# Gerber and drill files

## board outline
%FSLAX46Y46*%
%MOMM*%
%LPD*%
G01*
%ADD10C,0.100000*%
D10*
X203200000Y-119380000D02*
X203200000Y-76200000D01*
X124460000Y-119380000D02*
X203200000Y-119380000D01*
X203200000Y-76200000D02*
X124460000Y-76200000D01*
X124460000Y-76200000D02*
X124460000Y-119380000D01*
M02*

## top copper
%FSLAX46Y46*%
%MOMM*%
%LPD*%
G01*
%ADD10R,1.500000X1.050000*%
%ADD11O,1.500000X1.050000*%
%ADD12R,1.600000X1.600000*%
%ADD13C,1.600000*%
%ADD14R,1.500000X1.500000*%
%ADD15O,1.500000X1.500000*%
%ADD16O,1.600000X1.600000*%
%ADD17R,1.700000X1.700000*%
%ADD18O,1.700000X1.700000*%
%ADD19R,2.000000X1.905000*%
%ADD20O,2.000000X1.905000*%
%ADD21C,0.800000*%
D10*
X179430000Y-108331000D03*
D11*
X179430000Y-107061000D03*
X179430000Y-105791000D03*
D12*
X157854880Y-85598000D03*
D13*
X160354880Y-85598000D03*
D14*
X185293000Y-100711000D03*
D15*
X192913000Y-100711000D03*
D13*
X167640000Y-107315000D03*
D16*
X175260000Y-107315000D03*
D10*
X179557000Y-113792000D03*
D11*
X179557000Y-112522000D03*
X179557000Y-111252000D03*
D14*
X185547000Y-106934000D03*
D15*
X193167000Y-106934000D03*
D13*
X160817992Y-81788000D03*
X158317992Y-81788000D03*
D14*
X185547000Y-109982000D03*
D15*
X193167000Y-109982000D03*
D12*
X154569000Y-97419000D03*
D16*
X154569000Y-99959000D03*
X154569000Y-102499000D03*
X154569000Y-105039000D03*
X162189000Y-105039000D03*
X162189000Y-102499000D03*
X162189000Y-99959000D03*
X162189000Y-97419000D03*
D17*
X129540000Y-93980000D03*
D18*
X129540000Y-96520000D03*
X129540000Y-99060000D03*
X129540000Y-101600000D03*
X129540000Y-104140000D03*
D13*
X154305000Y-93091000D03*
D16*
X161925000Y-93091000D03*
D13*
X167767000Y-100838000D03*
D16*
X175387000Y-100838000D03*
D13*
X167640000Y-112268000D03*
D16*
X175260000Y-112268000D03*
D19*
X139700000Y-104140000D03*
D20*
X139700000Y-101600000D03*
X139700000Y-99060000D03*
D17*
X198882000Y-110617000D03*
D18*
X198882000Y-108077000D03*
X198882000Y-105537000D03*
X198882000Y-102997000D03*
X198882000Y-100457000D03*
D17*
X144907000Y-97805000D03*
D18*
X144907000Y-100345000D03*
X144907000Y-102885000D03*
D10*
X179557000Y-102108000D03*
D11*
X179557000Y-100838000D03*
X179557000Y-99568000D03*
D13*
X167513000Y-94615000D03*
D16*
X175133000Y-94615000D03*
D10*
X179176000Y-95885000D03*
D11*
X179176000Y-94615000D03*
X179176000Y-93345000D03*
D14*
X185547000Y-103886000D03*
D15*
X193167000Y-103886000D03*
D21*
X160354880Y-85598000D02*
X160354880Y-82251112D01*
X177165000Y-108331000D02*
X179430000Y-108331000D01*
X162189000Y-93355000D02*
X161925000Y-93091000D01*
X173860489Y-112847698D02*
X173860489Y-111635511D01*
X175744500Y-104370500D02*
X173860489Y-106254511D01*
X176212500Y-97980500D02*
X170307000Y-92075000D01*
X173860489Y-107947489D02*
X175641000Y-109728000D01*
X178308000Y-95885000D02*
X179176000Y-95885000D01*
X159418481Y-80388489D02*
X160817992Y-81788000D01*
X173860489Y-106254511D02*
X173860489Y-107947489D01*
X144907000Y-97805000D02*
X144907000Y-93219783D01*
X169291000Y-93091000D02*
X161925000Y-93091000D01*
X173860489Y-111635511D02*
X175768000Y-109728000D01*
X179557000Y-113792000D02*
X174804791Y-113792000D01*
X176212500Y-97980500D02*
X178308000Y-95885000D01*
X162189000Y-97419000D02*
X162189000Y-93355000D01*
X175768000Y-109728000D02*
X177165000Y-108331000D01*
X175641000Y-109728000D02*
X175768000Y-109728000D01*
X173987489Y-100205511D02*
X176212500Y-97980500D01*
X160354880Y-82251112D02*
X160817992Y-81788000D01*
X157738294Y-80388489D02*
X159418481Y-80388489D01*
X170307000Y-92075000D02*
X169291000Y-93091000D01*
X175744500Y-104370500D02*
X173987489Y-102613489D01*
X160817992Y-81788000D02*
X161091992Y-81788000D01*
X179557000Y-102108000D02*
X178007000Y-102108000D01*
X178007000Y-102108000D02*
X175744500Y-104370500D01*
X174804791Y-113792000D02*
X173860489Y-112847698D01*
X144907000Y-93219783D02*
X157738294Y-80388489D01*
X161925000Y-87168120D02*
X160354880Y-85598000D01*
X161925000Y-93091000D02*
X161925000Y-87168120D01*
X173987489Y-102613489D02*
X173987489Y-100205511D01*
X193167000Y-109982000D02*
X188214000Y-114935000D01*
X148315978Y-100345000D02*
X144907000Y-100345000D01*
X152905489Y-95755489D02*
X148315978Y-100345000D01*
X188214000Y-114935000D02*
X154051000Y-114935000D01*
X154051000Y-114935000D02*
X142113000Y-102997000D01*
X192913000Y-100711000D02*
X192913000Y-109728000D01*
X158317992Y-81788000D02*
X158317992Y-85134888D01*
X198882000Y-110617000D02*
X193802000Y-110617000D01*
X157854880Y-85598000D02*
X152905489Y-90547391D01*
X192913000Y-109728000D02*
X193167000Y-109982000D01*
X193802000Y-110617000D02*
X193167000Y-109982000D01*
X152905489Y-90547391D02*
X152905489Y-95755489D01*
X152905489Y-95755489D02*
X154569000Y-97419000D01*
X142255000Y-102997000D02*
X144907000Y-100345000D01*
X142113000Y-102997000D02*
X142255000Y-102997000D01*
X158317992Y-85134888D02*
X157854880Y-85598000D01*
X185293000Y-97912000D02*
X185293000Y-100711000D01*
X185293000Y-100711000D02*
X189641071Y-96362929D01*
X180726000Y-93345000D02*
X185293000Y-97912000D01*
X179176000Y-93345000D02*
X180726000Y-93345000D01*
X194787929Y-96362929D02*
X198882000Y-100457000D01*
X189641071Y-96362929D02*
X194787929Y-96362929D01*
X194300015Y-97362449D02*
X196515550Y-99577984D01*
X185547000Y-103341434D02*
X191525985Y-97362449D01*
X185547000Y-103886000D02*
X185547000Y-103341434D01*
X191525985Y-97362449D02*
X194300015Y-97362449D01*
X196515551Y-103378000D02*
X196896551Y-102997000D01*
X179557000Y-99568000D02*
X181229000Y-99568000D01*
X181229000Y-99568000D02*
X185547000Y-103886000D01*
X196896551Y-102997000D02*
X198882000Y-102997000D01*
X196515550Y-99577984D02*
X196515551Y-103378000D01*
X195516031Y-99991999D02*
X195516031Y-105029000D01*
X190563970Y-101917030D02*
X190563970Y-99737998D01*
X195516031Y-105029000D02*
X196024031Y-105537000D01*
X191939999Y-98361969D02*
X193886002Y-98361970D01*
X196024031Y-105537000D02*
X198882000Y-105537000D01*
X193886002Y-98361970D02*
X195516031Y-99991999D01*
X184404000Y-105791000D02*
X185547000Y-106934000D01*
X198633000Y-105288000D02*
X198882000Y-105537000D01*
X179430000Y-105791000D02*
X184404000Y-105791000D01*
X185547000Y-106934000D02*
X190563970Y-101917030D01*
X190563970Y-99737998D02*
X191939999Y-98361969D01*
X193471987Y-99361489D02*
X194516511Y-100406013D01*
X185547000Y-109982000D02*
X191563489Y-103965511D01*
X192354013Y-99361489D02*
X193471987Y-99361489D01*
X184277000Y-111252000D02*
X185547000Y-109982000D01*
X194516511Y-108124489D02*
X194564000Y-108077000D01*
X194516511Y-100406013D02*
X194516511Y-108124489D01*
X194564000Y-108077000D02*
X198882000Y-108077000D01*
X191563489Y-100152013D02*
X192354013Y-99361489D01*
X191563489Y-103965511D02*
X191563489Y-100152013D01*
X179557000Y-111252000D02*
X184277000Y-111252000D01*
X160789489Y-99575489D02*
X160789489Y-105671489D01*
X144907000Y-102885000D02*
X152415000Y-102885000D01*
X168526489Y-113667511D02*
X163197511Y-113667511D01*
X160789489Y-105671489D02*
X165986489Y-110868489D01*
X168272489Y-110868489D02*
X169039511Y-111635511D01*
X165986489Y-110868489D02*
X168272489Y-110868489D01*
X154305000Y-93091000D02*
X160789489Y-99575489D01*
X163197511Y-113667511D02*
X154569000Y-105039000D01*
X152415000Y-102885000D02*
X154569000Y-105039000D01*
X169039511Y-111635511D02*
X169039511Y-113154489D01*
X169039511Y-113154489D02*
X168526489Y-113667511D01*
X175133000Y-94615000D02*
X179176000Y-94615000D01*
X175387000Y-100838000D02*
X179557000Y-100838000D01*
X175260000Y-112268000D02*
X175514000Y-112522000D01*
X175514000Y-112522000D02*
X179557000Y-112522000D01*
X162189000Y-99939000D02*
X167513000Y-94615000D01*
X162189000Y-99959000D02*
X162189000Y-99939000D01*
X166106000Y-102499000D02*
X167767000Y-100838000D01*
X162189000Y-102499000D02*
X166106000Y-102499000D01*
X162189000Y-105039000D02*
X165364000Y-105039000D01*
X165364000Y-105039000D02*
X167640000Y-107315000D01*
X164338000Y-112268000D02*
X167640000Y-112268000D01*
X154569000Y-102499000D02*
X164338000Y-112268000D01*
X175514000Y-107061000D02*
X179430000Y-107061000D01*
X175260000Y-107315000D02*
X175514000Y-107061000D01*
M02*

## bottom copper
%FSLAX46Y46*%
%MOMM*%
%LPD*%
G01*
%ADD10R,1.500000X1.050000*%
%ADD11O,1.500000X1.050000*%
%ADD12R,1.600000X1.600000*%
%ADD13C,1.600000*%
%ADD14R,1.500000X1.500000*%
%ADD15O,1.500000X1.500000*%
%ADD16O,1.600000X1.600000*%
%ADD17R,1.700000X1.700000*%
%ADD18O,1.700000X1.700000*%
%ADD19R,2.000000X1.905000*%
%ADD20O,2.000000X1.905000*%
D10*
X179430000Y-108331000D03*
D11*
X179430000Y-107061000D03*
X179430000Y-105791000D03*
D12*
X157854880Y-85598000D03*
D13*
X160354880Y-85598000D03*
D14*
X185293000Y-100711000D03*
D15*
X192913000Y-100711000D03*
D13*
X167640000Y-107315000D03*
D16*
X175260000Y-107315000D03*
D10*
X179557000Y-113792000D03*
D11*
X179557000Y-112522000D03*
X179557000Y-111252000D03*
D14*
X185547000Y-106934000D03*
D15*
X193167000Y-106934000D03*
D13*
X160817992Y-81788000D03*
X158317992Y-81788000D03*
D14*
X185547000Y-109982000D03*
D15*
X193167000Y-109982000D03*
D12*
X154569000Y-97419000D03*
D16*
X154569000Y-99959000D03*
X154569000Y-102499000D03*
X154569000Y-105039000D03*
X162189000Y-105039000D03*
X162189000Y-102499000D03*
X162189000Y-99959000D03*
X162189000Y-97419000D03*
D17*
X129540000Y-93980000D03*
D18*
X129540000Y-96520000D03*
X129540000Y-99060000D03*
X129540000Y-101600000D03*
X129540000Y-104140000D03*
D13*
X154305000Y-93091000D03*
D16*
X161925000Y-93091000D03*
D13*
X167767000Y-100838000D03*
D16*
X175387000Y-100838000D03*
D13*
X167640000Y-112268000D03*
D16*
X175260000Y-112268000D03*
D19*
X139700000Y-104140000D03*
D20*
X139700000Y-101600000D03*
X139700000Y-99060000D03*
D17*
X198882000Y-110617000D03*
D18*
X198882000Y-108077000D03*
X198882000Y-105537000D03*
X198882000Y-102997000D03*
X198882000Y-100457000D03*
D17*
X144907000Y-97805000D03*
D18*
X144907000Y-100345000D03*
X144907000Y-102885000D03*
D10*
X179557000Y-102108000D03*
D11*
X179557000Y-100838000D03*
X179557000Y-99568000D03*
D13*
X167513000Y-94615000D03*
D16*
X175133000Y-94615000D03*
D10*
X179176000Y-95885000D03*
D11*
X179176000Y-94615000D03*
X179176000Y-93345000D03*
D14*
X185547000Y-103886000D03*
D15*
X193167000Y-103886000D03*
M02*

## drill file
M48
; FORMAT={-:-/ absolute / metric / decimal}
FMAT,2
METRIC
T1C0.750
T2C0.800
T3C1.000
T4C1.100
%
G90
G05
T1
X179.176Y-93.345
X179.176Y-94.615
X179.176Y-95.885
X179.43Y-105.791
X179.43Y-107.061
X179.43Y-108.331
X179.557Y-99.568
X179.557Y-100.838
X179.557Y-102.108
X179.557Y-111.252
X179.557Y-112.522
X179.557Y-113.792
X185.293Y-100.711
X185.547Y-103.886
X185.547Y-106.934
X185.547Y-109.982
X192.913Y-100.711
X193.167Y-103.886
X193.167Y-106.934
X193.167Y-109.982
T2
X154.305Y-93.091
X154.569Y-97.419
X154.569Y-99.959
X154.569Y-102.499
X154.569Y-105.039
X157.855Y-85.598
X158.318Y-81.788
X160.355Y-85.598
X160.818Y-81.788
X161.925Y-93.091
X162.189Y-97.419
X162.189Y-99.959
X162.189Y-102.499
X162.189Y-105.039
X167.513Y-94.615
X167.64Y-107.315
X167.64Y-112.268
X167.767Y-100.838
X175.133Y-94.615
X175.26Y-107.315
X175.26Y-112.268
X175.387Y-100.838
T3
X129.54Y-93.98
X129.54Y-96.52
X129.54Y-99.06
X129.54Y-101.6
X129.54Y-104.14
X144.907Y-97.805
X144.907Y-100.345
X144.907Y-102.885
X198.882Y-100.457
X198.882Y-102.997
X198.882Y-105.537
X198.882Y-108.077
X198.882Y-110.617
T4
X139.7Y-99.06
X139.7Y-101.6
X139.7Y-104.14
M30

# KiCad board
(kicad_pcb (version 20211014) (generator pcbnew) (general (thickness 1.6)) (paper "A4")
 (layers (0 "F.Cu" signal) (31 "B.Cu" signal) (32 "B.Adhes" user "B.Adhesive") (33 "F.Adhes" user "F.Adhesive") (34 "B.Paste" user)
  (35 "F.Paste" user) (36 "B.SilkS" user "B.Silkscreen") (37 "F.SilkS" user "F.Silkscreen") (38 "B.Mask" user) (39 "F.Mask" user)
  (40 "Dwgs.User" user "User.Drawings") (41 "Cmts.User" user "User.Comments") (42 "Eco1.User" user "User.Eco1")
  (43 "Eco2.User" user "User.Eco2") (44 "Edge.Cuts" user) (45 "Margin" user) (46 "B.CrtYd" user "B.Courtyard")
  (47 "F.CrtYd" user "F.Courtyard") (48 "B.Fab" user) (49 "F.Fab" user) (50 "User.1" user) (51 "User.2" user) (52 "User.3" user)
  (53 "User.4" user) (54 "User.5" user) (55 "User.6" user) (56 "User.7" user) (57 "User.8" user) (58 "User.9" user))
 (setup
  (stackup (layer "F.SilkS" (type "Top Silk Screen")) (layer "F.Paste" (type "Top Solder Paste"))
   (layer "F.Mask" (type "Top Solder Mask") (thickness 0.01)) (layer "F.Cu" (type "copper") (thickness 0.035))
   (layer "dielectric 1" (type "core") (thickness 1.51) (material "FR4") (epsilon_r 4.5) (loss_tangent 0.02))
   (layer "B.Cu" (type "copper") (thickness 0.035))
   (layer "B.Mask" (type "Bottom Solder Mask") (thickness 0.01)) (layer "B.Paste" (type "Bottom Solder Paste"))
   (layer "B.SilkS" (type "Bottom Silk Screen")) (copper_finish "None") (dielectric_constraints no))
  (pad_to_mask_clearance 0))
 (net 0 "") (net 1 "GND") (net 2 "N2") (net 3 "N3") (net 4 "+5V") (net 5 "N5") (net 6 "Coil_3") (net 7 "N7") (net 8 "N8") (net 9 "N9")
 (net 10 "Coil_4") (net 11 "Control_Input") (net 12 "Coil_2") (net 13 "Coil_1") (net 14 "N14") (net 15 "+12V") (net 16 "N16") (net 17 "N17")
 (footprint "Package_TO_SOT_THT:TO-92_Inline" (layer "F.Cu") (at 179.43 108.331 90)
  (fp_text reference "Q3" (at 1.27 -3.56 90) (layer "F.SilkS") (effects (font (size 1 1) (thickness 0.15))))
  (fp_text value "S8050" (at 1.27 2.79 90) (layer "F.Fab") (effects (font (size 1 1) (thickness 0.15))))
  (pad "1" thru_hole rect (at 0 0 90) (size 1.05 1.5) (drill 0.75) (layers *.Cu *.Mask) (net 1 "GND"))
  (pad "2" thru_hole oval (at 1.27 0 90) (size 1.05 1.5) (drill 0.75) (layers *.Cu *.Mask) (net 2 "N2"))
  (pad "3" thru_hole oval (at 2.54 0 90) (size 1.05 1.5) (drill 0.75) (layers *.Cu *.Mask) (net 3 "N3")))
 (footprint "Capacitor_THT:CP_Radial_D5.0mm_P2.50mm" (layer "F.Cu") (at 157.85488 85.598)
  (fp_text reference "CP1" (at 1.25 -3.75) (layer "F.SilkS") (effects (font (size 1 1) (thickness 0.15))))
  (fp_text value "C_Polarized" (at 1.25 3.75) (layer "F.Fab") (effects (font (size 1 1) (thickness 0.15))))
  (pad "1" thru_hole rect (at 0 0) (size 1.6 1.6) (drill 0.8) (layers *.Cu *.Mask) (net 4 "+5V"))
  (pad "2" thru_hole circle (at 2.5 0) (size 1.6 1.6) (drill 0.8) (layers *.Cu *.Mask) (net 1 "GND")))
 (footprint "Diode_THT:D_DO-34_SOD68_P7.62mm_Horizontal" (layer "F.Cu") (at 185.293 100.711)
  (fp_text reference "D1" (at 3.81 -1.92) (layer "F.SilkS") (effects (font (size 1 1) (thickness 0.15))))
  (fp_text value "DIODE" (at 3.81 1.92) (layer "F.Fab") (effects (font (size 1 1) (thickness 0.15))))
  (pad "1" thru_hole rect (at 0 0) (size 1.5 1.5) (drill 0.75) (layers *.Cu *.Mask) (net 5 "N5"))
  (pad "2" thru_hole oval (at 7.62 0) (size 1.5 1.5) (drill 0.75) (layers *.Cu *.Mask) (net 4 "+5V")))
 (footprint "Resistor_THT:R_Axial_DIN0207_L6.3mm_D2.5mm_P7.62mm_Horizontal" (layer "F.Cu") (at 167.64 107.315)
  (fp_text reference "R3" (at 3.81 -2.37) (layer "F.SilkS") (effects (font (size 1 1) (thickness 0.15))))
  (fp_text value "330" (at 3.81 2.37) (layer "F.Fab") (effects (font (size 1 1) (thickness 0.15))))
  (pad "1" thru_hole circle (at 0 0) (size 1.6 1.6) (drill 0.8) (layers *.Cu *.Mask) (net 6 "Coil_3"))
  (pad "2" thru_hole oval (at 7.62 0) (size 1.6 1.6) (drill 0.8) (layers *.Cu *.Mask) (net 2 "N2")))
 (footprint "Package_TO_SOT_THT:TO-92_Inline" (layer "F.Cu") (at 179.557 113.792 90)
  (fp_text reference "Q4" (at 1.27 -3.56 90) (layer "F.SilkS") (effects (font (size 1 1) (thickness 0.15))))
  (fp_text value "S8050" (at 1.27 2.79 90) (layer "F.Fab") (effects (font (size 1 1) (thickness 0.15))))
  (pad "1" thru_hole rect (at 0 0 90) (size 1.05 1.5) (drill 0.75) (layers *.Cu *.Mask) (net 1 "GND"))
  (pad "2" thru_hole oval (at 1.27 0 90) (size 1.05 1.5) (drill 0.75) (layers *.Cu *.Mask) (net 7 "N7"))
  (pad "3" thru_hole oval (at 2.54 0 90) (size 1.05 1.5) (drill 0.75) (layers *.Cu *.Mask) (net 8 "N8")))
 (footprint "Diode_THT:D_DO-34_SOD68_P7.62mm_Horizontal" (layer "F.Cu") (at 185.547 106.934)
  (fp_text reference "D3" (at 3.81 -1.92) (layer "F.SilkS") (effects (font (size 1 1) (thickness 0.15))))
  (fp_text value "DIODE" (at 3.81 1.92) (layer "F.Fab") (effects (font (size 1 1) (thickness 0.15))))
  (pad "1" thru_hole rect (at 0 0) (size 1.5 1.5) (drill 0.75) (layers *.Cu *.Mask) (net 3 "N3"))
  (pad "2" thru_hole oval (at 7.62 0) (size 1.5 1.5) (drill 0.75) (layers *.Cu *.Mask) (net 4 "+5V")))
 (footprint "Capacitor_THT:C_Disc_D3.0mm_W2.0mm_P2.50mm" (layer "F.Cu") (at 160.817992 81.788 180)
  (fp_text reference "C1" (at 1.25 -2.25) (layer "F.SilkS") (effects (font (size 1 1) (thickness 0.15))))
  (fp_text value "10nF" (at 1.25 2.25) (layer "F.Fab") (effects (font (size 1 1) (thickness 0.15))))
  (pad "1" thru_hole circle (at 0 0 180) (size 1.6 1.6) (drill 0.8) (layers *.Cu *.Mask) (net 1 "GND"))
  (pad "2" thru_hole circle (at 2.5 0 180) (size 1.6 1.6) (drill 0.8) (layers *.Cu *.Mask) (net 4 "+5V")))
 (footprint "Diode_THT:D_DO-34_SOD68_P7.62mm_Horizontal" (layer "F.Cu") (at 185.547 109.982)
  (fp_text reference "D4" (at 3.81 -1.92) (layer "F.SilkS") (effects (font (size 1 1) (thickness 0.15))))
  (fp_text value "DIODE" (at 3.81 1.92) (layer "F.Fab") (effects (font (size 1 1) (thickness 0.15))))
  (pad "1" thru_hole rect (at 0 0) (size 1.5 1.5) (drill 0.75) (layers *.Cu *.Mask) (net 8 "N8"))
  (pad "2" thru_hole oval (at 7.62 0) (size 1.5 1.5) (drill 0.75) (layers *.Cu *.Mask) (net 4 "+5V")))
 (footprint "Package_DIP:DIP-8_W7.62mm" (layer "F.Cu") (at 154.569 97.419)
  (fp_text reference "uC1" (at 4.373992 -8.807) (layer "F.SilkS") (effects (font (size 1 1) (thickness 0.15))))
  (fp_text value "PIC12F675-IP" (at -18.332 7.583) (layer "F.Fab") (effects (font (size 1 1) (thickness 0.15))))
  (pad "1" thru_hole rect (at 0 0) (size 1.6 1.6) (drill 0.8) (layers *.Cu *.Mask) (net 4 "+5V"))
  (pad "2" thru_hole oval (at 0 2.54) (size 1.6 1.6) (drill 0.8) (layers *.Cu *.Mask) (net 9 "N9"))
  (pad "3" thru_hole oval (at 0 5.08) (size 1.6 1.6) (drill 0.8) (layers *.Cu *.Mask) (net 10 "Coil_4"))
  (pad "4" thru_hole oval (at 0 7.62) (size 1.6 1.6) (drill 0.8) (layers *.Cu *.Mask) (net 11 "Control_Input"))
  (pad "5" thru_hole oval (at 7.62 7.62) (size 1.6 1.6) (drill 0.8) (layers *.Cu *.Mask) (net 6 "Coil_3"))
  (pad "6" thru_hole oval (at 7.62 5.08) (size 1.6 1.6) (drill 0.8) (layers *.Cu *.Mask) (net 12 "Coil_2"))
  (pad "7" thru_hole oval (at 7.62 2.54) (size 1.6 1.6) (drill 0.8) (layers *.Cu *.Mask) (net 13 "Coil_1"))
  (pad "8" thru_hole oval (at 7.62 0) (size 1.6 1.6) (drill 0.8) (layers *.Cu *.Mask) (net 1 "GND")))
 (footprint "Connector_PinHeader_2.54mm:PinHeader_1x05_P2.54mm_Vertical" (layer "F.Cu") (at 129.54 93.98)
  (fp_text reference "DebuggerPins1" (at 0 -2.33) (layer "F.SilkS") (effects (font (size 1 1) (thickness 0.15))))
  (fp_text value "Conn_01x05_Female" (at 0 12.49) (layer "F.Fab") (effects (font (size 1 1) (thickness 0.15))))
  (pad "1" thru_hole rect (at 0 0) (size 1.7 1.7) (drill 1) (layers *.Cu *.Mask) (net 11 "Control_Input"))
  (pad "2" thru_hole oval (at 0 2.54) (size 1.7 1.7) (drill 1) (layers *.Cu *.Mask) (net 4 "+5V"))
  (pad "3" thru_hole oval (at 0 5.08) (size 1.7 1.7) (drill 1) (layers *.Cu *.Mask) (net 1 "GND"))
  (pad "4" thru_hole oval (at 0 7.62) (size 1.7 1.7) (drill 1) (layers *.Cu *.Mask) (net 13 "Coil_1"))
  (pad "5" thru_hole oval (at 0 10.16) (size 1.7 1.7) (drill 1) (layers *.Cu *.Mask) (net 12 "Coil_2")))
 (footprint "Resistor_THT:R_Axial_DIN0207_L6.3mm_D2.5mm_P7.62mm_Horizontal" (layer "F.Cu") (at 154.305 93.091)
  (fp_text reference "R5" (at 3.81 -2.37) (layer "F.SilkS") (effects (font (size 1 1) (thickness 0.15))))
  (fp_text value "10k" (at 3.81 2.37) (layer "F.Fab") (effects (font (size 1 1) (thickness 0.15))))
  (pad "1" thru_hole circle (at 0 0) (size 1.6 1.6) (drill 0.8) (layers *.Cu *.Mask) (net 1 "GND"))
  (pad "2" thru_hole oval (at 7.62 0) (size 1.6 1.6) (drill 0.8) (layers *.Cu *.Mask) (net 11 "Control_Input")))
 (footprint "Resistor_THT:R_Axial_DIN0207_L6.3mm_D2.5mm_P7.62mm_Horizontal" (layer "F.Cu") (at 167.767 100.838)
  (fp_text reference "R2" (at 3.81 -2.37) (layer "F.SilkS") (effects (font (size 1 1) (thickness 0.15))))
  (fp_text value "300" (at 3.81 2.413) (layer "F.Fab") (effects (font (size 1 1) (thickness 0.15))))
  (pad "1" thru_hole circle (at 0 0) (size 1.6 1.6) (drill 0.8) (layers *.Cu *.Mask) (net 12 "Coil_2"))
  (pad "2" thru_hole oval (at 7.62 0) (size 1.6 1.6) (drill 0.8) (layers *.Cu *.Mask) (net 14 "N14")))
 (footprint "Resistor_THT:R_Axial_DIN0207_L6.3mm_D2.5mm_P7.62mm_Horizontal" (layer "F.Cu") (at 167.64 112.268)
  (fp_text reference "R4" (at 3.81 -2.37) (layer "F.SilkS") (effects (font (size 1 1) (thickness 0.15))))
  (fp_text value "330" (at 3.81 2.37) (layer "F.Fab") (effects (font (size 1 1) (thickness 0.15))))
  (pad "1" thru_hole circle (at 0 0) (size 1.6 1.6) (drill 0.8) (layers *.Cu *.Mask) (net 10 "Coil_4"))
  (pad "2" thru_hole oval (at 7.62 0) (size 1.6 1.6) (drill 0.8) (layers *.Cu *.Mask) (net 7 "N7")))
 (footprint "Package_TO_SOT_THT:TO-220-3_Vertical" (layer "F.Cu") (at 139.7 104.14 90)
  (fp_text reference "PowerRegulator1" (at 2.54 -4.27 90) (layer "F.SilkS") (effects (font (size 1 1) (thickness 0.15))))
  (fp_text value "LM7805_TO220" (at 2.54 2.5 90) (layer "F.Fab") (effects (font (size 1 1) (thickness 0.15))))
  (pad "1" thru_hole rect (at 0 0 90) (size 1.905 2) (drill 1.1) (layers *.Cu *.Mask) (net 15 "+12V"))
  (pad "2" thru_hole oval (at 2.54 0 90) (size 1.905 2) (drill 1.1) (layers *.Cu *.Mask) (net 1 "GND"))
  (pad "3" thru_hole oval (at 5.08 0 90) (size 1.905 2) (drill 1.1) (layers *.Cu *.Mask) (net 4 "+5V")))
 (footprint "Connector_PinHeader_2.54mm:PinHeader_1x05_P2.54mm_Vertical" (layer "F.Cu") (at 198.882 110.617 180)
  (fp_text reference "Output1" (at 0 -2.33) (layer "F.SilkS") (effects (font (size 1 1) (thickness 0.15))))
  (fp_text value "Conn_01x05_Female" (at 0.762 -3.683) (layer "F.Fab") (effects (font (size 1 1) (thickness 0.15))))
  (pad "1" thru_hole rect (at 0 0 180) (size 1.7 1.7) (drill 1) (layers *.Cu *.Mask) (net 4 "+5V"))
  (pad "2" thru_hole oval (at 0 2.54 180) (size 1.7 1.7) (drill 1) (layers *.Cu *.Mask) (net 8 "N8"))
  (pad "3" thru_hole oval (at 0 5.08 180) (size 1.7 1.7) (drill 1) (layers *.Cu *.Mask) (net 3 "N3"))
  (pad "4" thru_hole oval (at 0 7.62 180) (size 1.7 1.7) (drill 1) (layers *.Cu *.Mask) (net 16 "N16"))
  (pad "5" thru_hole oval (at 0 10.16 180) (size 1.7 1.7) (drill 1) (layers *.Cu *.Mask) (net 5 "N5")))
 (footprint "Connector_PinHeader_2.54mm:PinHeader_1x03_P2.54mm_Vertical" (layer "F.Cu") (at 144.907 97.805)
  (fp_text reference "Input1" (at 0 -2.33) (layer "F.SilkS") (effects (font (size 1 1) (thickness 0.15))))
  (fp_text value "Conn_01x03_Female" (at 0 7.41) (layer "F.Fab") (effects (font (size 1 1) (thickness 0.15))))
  (pad "1" thru_hole rect (at 0 0) (size 1.7 1.7) (drill 1) (layers *.Cu *.Mask) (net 1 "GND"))
  (pad "2" thru_hole oval (at 0 2.54) (size 1.7 1.7) (drill 1) (layers *.Cu *.Mask) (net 15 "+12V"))
  (pad "3" thru_hole oval (at 0 5.08) (size 1.7 1.7) (drill 1) (layers *.Cu *.Mask) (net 11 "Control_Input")))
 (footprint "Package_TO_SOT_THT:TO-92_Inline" (layer "F.Cu") (at 179.557 102.108 90)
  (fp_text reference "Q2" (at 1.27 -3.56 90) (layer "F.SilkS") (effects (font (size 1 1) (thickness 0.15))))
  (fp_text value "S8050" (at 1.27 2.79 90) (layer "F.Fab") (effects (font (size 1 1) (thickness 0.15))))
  (pad "1" thru_hole rect (at 0 0 90) (size 1.05 1.5) (drill 0.75) (layers *.Cu *.Mask) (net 1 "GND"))
  (pad "2" thru_hole oval (at 1.27 0 90) (size 1.05 1.5) (drill 0.75) (layers *.Cu *.Mask) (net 14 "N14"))
  (pad "3" thru_hole oval (at 2.54 0 90) (size 1.05 1.5) (drill 0.75) (layers *.Cu *.Mask) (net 16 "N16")))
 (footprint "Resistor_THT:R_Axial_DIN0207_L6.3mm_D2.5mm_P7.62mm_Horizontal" (layer "F.Cu") (at 167.513 94.615)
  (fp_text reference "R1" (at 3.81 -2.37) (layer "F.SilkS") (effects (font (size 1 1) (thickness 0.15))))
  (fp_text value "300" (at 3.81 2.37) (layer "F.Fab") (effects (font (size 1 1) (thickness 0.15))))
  (pad "1" thru_hole circle (at 0 0) (size 1.6 1.6) (drill 0.8) (layers *.Cu *.Mask) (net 13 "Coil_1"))
  (pad "2" thru_hole oval (at 7.62 0) (size 1.6 1.6) (drill 0.8) (layers *.Cu *.Mask) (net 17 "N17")))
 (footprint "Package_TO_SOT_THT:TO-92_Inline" (layer "F.Cu") (at 179.176 95.885 90)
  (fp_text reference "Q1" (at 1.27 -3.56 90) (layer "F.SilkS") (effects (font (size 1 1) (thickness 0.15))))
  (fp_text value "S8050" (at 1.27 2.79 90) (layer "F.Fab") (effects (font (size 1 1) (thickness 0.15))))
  (pad "1" thru_hole rect (at 0 0 90) (size 1.05 1.5) (drill 0.75) (layers *.Cu *.Mask) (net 1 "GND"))
  (pad "2" thru_hole oval (at 1.27 0 90) (size 1.05 1.5) (drill 0.75) (layers *.Cu *.Mask) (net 17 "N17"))
  (pad "3" thru_hole oval (at 2.54 0 90) (size 1.05 1.5) (drill 0.75) (layers *.Cu *.Mask) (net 5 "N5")))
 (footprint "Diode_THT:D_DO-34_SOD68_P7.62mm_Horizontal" (layer "F.Cu") (at 185.547 103.886)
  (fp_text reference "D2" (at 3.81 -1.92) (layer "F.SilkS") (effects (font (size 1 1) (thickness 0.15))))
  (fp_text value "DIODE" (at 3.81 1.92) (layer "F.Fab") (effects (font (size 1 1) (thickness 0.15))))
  (pad "1" thru_hole rect (at 0 0) (size 1.5 1.5) (drill 0.75) (layers *.Cu *.Mask) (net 16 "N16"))
  (pad "2" thru_hole oval (at 7.62 0) (size 1.5 1.5) (drill 0.75) (layers *.Cu *.Mask) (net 4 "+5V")))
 (gr_line (start 203.2 119.38) (end 203.2 76.2) (layer "Edge.Cuts") (width 0.1))
 (gr_line (start 124.46 119.38) (end 203.2 119.38) (layer "Edge.Cuts") (width 0.1))
 (gr_line (start 203.2 76.2) (end 124.46 76.2) (layer "Edge.Cuts") (width 0.1))
 (gr_line (start 124.46 76.2) (end 124.46 119.38) (layer "Edge.Cuts") (width 0.1))
 (segment (start 160.35488 85.598) (end 160.35488 82.251112) (width 0.8) (layer "F.Cu") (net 1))
 (segment (start 177.165 108.331) (end 179.43 108.331) (width 0.8) (layer "F.Cu") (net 1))
 (segment (start 162.189 93.355) (end 161.925 93.091) (width 0.8) (layer "F.Cu") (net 1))
 (segment (start 173.860489 112.847698) (end 173.860489 111.635511) (width 0.8) (layer "F.Cu") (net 1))
 (segment (start 175.7445 104.3705) (end 173.860489 106.254511) (width 0.8) (layer "F.Cu") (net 1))
 (segment (start 176.2125 97.9805) (end 170.307 92.075) (width 0.8) (layer "F.Cu") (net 1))
 (segment (start 173.860489 107.947489) (end 175.641 109.728) (width 0.8) (layer "F.Cu") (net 1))
 (segment (start 178.308 95.885) (end 179.176 95.885) (width 0.8) (layer "F.Cu") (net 1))
 (segment (start 159.418481 80.388489) (end 160.817992 81.788) (width 0.8) (layer "F.Cu") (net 1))
 (segment (start 173.860489 106.254511) (end 173.860489 107.947489) (width 0.8) (layer "F.Cu") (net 1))
 (segment (start 144.907 97.805) (end 144.907 93.219783) (width 0.8) (layer "F.Cu") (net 1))
 (segment (start 169.291 93.091) (end 161.925 93.091) (width 0.8) (layer "F.Cu") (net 1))
 (segment (start 173.860489 111.635511) (end 175.768 109.728) (width 0.8) (layer "F.Cu") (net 1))
 (segment (start 179.557 113.792) (end 174.804791 113.792) (width 0.8) (layer "F.Cu") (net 1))
 (segment (start 176.2125 97.9805) (end 178.308 95.885) (width 0.8) (layer "F.Cu") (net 1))
 (segment (start 162.189 97.419) (end 162.189 93.355) (width 0.8) (layer "F.Cu") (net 1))
 (segment (start 175.768 109.728) (end 177.165 108.331) (width 0.8) (layer "F.Cu") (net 1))
 (segment (start 175.641 109.728) (end 175.768 109.728) (width 0.8) (layer "F.Cu") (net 1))
 (segment (start 173.987489 100.205511) (end 176.2125 97.9805) (width 0.8) (layer "F.Cu") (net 1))
 (segment (start 160.35488 82.251112) (end 160.817992 81.788) (width 0.8) (layer "F.Cu") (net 1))
 (segment (start 157.738294 80.388489) (end 159.418481 80.388489) (width 0.8) (layer "F.Cu") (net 1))
 (segment (start 170.307 92.075) (end 169.291 93.091) (width 0.8) (layer "F.Cu") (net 1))
 (segment (start 175.7445 104.3705) (end 173.987489 102.613489) (width 0.8) (layer "F.Cu") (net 1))
 (segment (start 160.817992 81.788) (end 161.091992 81.788) (width 0.8) (layer "F.Cu") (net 1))
 (segment (start 179.557 102.108) (end 178.007 102.108) (width 0.8) (layer "F.Cu") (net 1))
 (segment (start 178.007 102.108) (end 175.7445 104.3705) (width 0.8) (layer "F.Cu") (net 1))
 (segment (start 174.804791 113.792) (end 173.860489 112.847698) (width 0.8) (layer "F.Cu") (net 1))
 (segment (start 144.907 93.219783) (end 157.738294 80.388489) (width 0.8) (layer "F.Cu") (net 1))
 (segment (start 161.925 87.16812) (end 160.35488 85.598) (width 0.8) (layer "F.Cu") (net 1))
 (segment (start 161.925 93.091) (end 161.925 87.16812) (width 0.8) (layer "F.Cu") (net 1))
 (segment (start 173.987489 102.613489) (end 173.987489 100.205511) (width 0.8) (layer "F.Cu") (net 1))
 (segment (start 193.167 109.982) (end 188.214 114.935) (width 0.8) (layer "F.Cu") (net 4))
 (segment (start 148.315978 100.345) (end 144.907 100.345) (width 0.8) (layer "F.Cu") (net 4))
 (segment (start 152.905489 95.755489) (end 148.315978 100.345) (width 0.8) (layer "F.Cu") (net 4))
 (segment (start 188.214 114.935) (end 154.051 114.935) (width 0.8) (layer "F.Cu") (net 4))
 (segment (start 154.051 114.935) (end 142.113 102.997) (width 0.8) (layer "F.Cu") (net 4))
 (segment (start 192.913 100.711) (end 192.913 109.728) (width 0.8) (layer "F.Cu") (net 4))
 (segment (start 158.317992 81.788) (end 158.317992 85.134888) (width 0.8) (layer "F.Cu") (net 4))
 (segment (start 198.882 110.617) (end 193.802 110.617) (width 0.8) (layer "F.Cu") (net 4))
 (segment (start 157.85488 85.598) (end 152.905489 90.547391) (width 0.8) (layer "F.Cu") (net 4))
 (segment (start 192.913 109.728) (end 193.167 109.982) (width 0.8) (layer "F.Cu") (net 4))
 (segment (start 193.802 110.617) (end 193.167 109.982) (width 0.8) (layer "F.Cu") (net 4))
 (segment (start 152.905489 90.547391) (end 152.905489 95.755489) (width 0.8) (layer "F.Cu") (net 4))
 (segment (start 152.905489 95.755489) (end 154.569 97.419) (width 0.8) (layer "F.Cu") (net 4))
 (segment (start 142.255 102.997) (end 144.907 100.345) (width 0.8) (layer "F.Cu") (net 4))
 (segment (start 142.113 102.997) (end 142.255 102.997) (width 0.8) (layer "F.Cu") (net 4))
 (segment (start 158.317992 85.134888) (end 157.85488 85.598) (width 0.8) (layer "F.Cu") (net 4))
 (segment (start 185.293 97.912) (end 185.293 100.711) (width 0.8) (layer "F.Cu") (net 5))
 (segment (start 185.293 100.711) (end 189.641071 96.362929) (width 0.8) (layer "F.Cu") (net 5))
 (segment (start 180.726 93.345) (end 185.293 97.912) (width 0.8) (layer "F.Cu") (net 5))
 (segment (start 179.176 93.345) (end 180.726 93.345) (width 0.8) (layer "F.Cu") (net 5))
 (segment (start 194.787929 96.362929) (end 198.882 100.457) (width 0.8) (layer "F.Cu") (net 5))
 (segment (start 189.641071 96.362929) (end 194.787929 96.362929) (width 0.8) (layer "F.Cu") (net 5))
 (segment (start 194.300015 97.362449) (end 196.51555 99.577984) (width 0.8) (layer "F.Cu") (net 16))
 (segment (start 185.547 103.341434) (end 191.525985 97.362449) (width 0.8) (layer "F.Cu") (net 16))
 (segment (start 185.547 103.886) (end 185.547 103.341434) (width 0.8) (layer "F.Cu") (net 16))
 (segment (start 191.525985 97.362449) (end 194.300015 97.362449) (width 0.8) (layer "F.Cu") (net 16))
 (segment (start 196.515551 103.378) (end 196.896551 102.997) (width 0.8) (layer "F.Cu") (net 16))
 (segment (start 179.557 99.568) (end 181.229 99.568) (width 0.8) (layer "F.Cu") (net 16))
 (segment (start 181.229 99.568) (end 185.547 103.886) (width 0.8) (layer "F.Cu") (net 16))
 (segment (start 196.896551 102.997) (end 198.882 102.997) (width 0.8) (layer "F.Cu") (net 16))
 (segment (start 196.51555 99.577984) (end 196.515551 103.378) (width 0.8) (layer "F.Cu") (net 16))
 (segment (start 195.516031 99.991999) (end 195.516031 105.029) (width 0.8) (layer "F.Cu") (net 3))
 (segment (start 190.56397 101.91703) (end 190.56397 99.737998) (width 0.8) (layer "F.Cu") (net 3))
 (segment (start 195.516031 105.029) (end 196.024031 105.537) (width 0.8) (layer "F.Cu") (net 3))
 (segment (start 191.939999 98.361969) (end 193.886002 98.36197) (width 0.8) (layer "F.Cu") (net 3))
 (segment (start 196.024031 105.537) (end 198.882 105.537) (width 0.8) (layer "F.Cu") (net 3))
 (segment (start 193.886002 98.36197) (end 195.516031 99.991999) (width 0.8) (layer "F.Cu") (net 3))
 (segment (start 184.404 105.791) (end 185.547 106.934) (width 0.8) (layer "F.Cu") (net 3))
 (segment (start 198.633 105.288) (end 198.882 105.537) (width 0.8) (layer "F.Cu") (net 3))
 (segment (start 179.43 105.791) (end 184.404 105.791) (width 0.8) (layer "F.Cu") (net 3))
 (segment (start 185.547 106.934) (end 190.56397 101.91703) (width 0.8) (layer "F.Cu") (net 3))
 (segment (start 190.56397 99.737998) (end 191.939999 98.361969) (width 0.8) (layer "F.Cu") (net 3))
 (segment (start 193.471987 99.361489) (end 194.516511 100.406013) (width 0.8) (layer "F.Cu") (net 8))
 (segment (start 185.547 109.982) (end 191.563489 103.965511) (width 0.8) (layer "F.Cu") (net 8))
 (segment (start 192.354013 99.361489) (end 193.471987 99.361489) (width 0.8) (layer "F.Cu") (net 8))
 (segment (start 184.277 111.252) (end 185.547 109.982) (width 0.8) (layer "F.Cu") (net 8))
 (segment (start 194.516511 108.124489) (end 194.564 108.077) (width 0.8) (layer "F.Cu") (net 8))
 (segment (start 194.516511 100.406013) (end 194.516511 108.124489) (width 0.8) (layer "F.Cu") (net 8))
 (segment (start 194.564 108.077) (end 198.882 108.077) (width 0.8) (layer "F.Cu") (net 8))
 (segment (start 191.563489 100.152013) (end 192.354013 99.361489) (width 0.8) (layer "F.Cu") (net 8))
 (segment (start 191.563489 103.965511) (end 191.563489 100.152013) (width 0.8) (layer "F.Cu") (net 8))
 (segment (start 179.557 111.252) (end 184.277 111.252) (width 0.8) (layer "F.Cu") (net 8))
 (segment (start 160.789489 99.575489) (end 160.789489 105.671489) (width 0.8) (layer "F.Cu") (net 11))
 (segment (start 144.907 102.885) (end 152.415 102.885) (width 0.8) (layer "F.Cu") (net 11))
 (segment (start 168.526489 113.667511) (end 163.197511 113.667511) (width 0.8) (layer "F.Cu") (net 11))
 (segment (start 160.789489 105.671489) (end 165.986489 110.868489) (width 0.8) (layer "F.Cu") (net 11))
 (segment (start 168.272489 110.868489) (end 169.039511 111.635511) (width 0.8) (layer "F.Cu") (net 11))
 (segment (start 165.986489 110.868489) (end 168.272489 110.868489) (width 0.8) (layer "F.Cu") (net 11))
 (segment (start 154.305 93.091) (end 160.789489 99.575489) (width 0.8) (layer "F.Cu") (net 11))
 (segment (start 163.197511 113.667511) (end 154.569 105.039) (width 0.8) (layer "F.Cu") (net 11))
 (segment (start 152.415 102.885) (end 154.569 105.039) (width 0.8) (layer "F.Cu") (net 11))
 (segment (start 169.039511 111.635511) (end 169.039511 113.154489) (width 0.8) (layer "F.Cu") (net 11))
 (segment (start 169.039511 113.154489) (end 168.526489 113.667511) (width 0.8) (layer "F.Cu") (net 11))
 (segment (start 175.133 94.615) (end 179.176 94.615) (width 0.8) (layer "F.Cu") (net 17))
 (segment (start 175.387 100.838) (end 179.557 100.838) (width 0.8) (layer "F.Cu") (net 14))
 (segment (start 175.26 112.268) (end 175.514 112.522) (width 0.8) (layer "F.Cu") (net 7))
 (segment (start 175.514 112.522) (end 179.557 112.522) (width 0.8) (layer "F.Cu") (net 7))
 (segment (start 162.189 99.939) (end 167.513 94.615) (width 0.8) (layer "F.Cu") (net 13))
 (segment (start 162.189 99.959) (end 162.189 99.939) (width 0.8) (layer "F.Cu") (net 13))
 (segment (start 166.106 102.499) (end 167.767 100.838) (width 0.8) (layer "F.Cu") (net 12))
 (segment (start 162.189 102.499) (end 166.106 102.499) (width 0.8) (layer "F.Cu") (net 12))
 (segment (start 162.189 105.039) (end 165.364 105.039) (width 0.8) (layer "F.Cu") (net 6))
 (segment (start 165.364 105.039) (end 167.64 107.315) (width 0.8) (layer "F.Cu") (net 6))
 (segment (start 164.338 112.268) (end 167.64 112.268) (width 0.8) (layer "F.Cu") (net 10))
 (segment (start 154.569 102.499) (end 164.338 112.268) (width 0.8) (layer "F.Cu") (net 10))
 (segment (start 175.514 107.061) (end 179.43 107.061) (width 0.8) (layer "F.Cu") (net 2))
 (segment (start 175.26 107.315) (end 175.514 107.061) (width 0.8) (layer "F.Cu") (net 2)))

